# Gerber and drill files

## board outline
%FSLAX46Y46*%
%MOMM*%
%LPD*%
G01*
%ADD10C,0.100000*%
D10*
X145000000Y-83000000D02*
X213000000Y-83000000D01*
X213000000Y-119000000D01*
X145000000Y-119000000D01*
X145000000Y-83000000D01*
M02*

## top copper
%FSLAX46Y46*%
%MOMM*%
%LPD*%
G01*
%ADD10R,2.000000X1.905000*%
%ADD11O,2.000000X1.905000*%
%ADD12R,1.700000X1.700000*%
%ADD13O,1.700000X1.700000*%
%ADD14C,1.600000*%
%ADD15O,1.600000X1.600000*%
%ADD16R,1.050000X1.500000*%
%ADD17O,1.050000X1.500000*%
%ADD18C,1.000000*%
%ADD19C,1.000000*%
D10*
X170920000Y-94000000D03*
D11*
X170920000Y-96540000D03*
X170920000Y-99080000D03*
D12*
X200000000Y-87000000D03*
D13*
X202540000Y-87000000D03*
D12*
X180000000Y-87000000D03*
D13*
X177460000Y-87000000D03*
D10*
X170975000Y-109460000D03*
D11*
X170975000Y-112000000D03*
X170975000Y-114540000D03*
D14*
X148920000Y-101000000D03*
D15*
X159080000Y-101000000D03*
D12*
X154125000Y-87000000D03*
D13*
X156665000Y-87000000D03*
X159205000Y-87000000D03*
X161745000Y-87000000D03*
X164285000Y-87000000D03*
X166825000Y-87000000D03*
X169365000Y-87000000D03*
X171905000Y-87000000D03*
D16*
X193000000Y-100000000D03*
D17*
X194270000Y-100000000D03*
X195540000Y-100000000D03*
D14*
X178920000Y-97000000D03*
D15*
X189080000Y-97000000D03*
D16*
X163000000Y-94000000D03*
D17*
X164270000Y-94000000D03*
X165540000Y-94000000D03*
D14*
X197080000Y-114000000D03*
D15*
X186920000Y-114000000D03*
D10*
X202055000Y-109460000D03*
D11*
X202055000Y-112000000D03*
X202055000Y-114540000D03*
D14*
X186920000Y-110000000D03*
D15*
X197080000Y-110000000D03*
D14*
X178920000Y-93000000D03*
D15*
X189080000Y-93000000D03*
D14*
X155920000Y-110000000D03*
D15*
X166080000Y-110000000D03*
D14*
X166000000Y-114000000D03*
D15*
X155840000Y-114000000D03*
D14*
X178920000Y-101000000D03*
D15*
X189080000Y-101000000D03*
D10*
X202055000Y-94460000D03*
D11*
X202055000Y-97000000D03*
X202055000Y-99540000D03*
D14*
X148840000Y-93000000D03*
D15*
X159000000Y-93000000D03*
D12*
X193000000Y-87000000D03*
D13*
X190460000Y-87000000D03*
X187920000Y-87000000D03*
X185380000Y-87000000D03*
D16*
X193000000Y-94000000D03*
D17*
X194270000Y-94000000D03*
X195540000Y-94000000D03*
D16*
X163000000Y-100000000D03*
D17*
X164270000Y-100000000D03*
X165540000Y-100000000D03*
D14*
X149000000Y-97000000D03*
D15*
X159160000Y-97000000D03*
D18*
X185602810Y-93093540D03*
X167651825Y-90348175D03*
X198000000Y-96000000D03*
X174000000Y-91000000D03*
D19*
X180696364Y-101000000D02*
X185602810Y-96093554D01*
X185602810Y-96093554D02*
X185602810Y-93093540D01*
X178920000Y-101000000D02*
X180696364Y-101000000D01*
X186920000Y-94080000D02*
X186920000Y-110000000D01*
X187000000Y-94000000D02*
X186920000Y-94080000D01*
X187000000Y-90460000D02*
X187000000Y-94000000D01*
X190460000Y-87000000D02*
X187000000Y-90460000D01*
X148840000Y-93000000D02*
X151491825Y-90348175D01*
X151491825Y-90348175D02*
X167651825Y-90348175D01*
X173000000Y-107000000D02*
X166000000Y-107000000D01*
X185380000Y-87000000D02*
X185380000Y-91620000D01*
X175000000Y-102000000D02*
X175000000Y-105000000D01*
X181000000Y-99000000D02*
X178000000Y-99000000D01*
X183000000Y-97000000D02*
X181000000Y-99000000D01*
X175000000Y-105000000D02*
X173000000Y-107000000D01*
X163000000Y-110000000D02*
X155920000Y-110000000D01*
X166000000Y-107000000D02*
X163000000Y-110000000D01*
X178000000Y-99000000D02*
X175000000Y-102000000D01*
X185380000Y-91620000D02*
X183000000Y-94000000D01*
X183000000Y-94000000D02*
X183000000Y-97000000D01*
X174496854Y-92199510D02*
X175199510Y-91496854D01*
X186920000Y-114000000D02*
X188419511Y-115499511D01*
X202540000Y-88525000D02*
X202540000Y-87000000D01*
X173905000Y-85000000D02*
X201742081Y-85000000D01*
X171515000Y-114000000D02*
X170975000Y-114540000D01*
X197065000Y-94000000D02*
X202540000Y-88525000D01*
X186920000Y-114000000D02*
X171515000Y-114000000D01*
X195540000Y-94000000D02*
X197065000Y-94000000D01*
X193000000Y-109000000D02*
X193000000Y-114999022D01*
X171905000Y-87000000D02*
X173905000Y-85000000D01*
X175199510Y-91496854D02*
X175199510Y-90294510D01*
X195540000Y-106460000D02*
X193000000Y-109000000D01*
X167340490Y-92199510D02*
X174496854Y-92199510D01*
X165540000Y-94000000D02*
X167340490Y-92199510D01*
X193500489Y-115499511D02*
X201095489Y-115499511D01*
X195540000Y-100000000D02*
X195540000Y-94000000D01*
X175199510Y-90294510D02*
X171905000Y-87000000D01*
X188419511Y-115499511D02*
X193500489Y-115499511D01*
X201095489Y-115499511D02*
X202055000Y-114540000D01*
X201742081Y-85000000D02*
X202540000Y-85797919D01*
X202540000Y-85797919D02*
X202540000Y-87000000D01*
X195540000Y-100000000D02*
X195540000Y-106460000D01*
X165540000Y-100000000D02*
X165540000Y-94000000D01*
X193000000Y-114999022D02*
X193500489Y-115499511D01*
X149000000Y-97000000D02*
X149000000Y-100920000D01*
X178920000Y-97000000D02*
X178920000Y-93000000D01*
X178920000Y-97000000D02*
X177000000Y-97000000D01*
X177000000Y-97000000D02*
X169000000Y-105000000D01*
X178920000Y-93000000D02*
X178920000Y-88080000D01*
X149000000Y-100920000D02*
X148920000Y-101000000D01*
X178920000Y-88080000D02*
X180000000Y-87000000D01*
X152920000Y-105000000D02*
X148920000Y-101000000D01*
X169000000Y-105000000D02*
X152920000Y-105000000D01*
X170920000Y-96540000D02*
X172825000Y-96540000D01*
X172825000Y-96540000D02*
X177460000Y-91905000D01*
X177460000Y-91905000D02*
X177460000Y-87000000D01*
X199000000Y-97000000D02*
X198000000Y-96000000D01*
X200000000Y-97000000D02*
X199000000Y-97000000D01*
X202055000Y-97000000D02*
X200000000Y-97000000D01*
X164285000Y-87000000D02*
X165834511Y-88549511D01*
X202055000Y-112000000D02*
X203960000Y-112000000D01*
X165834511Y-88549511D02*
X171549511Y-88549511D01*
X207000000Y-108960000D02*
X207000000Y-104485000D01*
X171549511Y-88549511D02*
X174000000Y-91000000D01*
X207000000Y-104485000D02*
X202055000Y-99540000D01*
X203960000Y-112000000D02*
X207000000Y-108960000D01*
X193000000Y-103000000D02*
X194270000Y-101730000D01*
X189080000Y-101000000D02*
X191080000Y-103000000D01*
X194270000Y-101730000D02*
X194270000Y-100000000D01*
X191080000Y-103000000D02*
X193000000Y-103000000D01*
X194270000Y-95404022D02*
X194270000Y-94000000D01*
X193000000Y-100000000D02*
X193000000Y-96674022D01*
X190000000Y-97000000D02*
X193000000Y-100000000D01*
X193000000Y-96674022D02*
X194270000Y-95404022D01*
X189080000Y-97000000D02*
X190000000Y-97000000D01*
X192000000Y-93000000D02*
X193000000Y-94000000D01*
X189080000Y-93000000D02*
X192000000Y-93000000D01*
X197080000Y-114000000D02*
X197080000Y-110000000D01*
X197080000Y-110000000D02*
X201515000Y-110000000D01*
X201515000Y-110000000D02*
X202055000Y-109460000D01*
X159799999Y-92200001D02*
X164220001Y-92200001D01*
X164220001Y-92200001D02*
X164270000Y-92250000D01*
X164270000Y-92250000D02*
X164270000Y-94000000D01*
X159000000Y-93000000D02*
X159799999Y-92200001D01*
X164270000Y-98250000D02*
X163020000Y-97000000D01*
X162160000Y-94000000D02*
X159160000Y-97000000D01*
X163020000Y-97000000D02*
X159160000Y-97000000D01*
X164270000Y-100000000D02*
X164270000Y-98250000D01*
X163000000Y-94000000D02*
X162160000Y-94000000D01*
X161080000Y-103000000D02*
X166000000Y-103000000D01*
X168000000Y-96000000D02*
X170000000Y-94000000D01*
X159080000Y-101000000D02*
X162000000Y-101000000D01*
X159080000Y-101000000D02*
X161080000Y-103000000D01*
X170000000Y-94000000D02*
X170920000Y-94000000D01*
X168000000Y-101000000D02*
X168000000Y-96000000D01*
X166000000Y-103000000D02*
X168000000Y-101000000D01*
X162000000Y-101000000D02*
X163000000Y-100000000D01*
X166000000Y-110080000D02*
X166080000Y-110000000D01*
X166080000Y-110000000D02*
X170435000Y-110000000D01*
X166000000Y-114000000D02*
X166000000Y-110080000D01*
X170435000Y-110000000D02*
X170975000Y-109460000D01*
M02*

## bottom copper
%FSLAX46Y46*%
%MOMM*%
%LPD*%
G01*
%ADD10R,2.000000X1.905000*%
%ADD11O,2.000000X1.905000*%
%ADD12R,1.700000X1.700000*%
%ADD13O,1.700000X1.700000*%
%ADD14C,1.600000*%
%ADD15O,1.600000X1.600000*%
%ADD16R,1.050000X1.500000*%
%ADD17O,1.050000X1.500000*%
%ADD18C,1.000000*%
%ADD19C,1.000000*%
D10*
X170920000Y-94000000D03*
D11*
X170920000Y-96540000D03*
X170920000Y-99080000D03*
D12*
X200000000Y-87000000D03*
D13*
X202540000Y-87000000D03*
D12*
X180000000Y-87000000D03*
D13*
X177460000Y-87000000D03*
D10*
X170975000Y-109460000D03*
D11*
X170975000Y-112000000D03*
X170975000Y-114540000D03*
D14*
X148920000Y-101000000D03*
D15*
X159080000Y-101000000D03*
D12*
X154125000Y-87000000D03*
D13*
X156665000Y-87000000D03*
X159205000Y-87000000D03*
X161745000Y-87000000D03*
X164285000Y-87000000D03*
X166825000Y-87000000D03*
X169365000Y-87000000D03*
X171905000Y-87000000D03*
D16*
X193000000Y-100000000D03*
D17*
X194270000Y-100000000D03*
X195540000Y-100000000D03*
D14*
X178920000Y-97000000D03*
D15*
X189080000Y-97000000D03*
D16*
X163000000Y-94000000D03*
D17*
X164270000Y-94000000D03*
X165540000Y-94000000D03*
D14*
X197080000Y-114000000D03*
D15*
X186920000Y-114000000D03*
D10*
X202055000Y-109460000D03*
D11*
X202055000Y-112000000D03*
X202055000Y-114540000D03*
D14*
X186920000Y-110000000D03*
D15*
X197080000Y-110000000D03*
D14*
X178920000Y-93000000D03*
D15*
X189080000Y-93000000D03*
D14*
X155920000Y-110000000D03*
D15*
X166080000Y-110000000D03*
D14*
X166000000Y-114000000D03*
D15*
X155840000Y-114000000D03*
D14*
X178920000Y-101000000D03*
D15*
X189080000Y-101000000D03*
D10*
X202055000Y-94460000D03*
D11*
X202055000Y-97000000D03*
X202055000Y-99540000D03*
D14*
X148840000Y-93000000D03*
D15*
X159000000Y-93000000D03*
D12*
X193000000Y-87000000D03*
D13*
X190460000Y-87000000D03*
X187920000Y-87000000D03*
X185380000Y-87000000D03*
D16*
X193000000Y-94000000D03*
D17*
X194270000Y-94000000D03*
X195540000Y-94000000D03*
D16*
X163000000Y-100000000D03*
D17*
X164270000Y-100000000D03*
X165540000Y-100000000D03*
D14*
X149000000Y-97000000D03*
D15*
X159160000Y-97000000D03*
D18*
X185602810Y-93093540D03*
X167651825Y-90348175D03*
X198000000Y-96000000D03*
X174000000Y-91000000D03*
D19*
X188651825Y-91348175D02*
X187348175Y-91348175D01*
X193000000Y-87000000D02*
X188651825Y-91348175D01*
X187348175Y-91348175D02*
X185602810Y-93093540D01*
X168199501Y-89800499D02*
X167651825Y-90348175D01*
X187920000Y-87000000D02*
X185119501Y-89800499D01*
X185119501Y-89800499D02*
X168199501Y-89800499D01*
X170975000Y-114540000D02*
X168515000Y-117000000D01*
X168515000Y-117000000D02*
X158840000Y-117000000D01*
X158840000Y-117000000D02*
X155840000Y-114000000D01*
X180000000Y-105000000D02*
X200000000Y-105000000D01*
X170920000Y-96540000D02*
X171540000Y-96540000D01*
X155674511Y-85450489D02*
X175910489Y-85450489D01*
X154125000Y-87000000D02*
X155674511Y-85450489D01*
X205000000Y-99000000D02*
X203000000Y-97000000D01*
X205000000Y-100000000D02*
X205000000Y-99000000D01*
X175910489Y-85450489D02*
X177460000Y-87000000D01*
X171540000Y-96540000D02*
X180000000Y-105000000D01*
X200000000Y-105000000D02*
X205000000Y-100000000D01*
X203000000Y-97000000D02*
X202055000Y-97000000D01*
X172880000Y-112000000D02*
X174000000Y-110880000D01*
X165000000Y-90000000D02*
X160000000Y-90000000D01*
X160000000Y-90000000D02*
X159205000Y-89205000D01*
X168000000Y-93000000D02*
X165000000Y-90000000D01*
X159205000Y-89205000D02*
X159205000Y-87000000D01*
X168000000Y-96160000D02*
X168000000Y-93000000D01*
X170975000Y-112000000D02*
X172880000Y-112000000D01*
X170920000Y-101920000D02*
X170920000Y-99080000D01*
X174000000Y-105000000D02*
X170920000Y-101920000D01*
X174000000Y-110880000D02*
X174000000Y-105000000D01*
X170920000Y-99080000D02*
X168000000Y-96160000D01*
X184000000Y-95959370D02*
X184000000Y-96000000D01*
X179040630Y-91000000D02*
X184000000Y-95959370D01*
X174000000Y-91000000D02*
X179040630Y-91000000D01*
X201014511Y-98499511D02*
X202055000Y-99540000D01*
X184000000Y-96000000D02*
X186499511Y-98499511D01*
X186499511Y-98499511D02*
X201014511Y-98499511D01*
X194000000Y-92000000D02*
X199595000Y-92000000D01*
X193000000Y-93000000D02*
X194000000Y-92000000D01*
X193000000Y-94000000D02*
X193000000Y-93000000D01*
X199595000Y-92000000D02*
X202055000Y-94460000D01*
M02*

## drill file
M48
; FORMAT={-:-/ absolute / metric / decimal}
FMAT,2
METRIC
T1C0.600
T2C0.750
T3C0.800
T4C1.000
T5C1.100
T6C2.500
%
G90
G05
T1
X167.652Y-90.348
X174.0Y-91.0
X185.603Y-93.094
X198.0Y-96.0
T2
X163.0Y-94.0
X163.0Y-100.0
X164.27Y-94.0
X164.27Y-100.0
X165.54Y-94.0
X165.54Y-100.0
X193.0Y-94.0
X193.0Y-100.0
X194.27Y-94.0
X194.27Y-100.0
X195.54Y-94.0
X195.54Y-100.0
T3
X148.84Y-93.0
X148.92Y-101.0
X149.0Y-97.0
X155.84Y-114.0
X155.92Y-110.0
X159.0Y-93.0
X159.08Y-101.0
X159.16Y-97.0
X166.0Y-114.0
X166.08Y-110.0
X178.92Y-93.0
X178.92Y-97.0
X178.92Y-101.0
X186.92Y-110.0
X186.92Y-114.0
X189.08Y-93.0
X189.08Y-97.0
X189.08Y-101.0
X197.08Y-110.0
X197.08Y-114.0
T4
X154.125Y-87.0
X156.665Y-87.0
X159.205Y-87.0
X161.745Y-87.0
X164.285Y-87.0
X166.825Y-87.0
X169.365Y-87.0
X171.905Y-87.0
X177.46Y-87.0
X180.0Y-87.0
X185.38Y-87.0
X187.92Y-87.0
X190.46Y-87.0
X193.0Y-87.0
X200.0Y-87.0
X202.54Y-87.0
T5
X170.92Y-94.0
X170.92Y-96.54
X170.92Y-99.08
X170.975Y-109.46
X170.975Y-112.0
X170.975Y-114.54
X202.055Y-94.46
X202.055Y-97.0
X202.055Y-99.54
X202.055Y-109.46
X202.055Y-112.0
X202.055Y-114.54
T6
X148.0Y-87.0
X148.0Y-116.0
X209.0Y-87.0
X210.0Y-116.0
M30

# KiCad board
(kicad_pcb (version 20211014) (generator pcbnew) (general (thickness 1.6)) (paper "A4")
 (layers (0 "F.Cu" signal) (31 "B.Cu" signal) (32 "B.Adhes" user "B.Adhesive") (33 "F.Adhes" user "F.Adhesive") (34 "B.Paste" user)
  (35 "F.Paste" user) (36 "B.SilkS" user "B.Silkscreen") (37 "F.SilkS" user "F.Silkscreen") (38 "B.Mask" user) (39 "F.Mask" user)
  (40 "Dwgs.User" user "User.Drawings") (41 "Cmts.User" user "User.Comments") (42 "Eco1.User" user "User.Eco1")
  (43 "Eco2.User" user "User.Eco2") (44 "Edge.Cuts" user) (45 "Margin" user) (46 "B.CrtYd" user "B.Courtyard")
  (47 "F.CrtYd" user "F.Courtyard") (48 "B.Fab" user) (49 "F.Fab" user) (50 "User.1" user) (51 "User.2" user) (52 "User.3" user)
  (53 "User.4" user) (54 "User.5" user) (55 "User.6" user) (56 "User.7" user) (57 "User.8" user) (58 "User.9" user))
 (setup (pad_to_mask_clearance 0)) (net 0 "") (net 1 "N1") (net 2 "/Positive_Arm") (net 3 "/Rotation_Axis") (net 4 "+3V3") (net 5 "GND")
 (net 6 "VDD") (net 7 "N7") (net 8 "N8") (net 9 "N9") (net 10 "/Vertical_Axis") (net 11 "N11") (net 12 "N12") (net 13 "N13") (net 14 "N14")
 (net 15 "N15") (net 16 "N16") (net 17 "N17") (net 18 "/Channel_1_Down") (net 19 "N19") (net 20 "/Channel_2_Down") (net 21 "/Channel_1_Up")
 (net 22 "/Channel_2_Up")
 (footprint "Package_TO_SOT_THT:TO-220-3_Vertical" (layer "F.Cu") (at 170.92 94 -90)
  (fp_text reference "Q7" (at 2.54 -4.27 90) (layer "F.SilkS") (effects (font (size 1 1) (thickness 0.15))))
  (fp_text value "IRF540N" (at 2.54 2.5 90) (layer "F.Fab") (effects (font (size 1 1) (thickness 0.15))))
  (pad "1" thru_hole rect locked (at 0 0 270) (size 1.905 2) (drill 1.1) (layers *.Cu *.Mask) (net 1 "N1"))
  (pad "2" thru_hole oval locked (at 2.54 0 270) (size 1.905 2) (drill 1.1) (layers *.Cu *.Mask) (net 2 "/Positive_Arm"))
  (pad "3" thru_hole oval locked (at 5.08 0 270) (size 1.905 2) (drill 1.1) (layers *.Cu *.Mask) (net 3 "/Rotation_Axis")))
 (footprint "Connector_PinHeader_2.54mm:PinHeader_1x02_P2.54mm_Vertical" (layer "F.Cu") (at 200 87 90)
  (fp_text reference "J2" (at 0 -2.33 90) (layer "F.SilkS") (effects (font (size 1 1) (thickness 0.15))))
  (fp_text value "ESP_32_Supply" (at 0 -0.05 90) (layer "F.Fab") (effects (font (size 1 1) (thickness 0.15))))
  (pad "1" thru_hole rect locked (at 0 0 90) (size 1.7 1.7) (drill 1) (layers *.Cu *.Mask) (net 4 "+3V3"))
  (pad "2" thru_hole oval locked (at 0 2.54 90) (size 1.7 1.7) (drill 1) (layers *.Cu *.Mask) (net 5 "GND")))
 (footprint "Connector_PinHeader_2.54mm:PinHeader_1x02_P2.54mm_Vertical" (layer "F.Cu") (at 180 87 -90)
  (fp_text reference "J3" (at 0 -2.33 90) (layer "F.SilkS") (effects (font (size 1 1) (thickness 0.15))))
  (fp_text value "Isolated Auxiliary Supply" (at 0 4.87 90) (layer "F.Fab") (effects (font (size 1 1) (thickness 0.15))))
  (pad "1" thru_hole rect locked (at 0 0 270) (size 1.7 1.7) (drill 1) (layers *.Cu *.Mask) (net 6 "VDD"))
  (pad "2" thru_hole oval locked (at 0 2.54 270) (size 1.7 1.7) (drill 1) (layers *.Cu *.Mask) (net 2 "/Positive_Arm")))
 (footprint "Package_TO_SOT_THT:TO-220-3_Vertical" (layer "F.Cu") (at 170.975 109.46 -90)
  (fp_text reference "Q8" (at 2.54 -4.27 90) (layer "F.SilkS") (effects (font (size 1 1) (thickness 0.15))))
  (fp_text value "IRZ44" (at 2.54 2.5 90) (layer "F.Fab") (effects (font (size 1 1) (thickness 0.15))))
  (pad "1" thru_hole rect locked (at 0 0 270) (size 1.905 2) (drill 1.1) (layers *.Cu *.Mask) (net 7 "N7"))
  (pad "2" thru_hole oval locked (at 2.54 0 270) (size 1.905 2) (drill 1.1) (layers *.Cu *.Mask) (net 3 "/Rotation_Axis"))
  (pad "3" thru_hole oval locked (at 5.08 0 270) (size 1.905 2) (drill 1.1) (layers *.Cu *.Mask) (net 5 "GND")))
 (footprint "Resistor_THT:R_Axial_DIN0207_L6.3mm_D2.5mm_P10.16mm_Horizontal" (layer "F.Cu") (at 148.92 101)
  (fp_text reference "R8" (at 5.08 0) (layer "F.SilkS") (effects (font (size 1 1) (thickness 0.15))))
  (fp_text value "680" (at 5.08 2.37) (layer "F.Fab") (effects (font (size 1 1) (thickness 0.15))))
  (pad "1" thru_hole circle locked (at 0 0) (size 1.6 1.6) (drill 0.8) (layers *.Cu *.Mask) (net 6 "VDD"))
  (pad "2" thru_hole oval locked (at 10.16 0) (size 1.6 1.6) (drill 0.8) (layers *.Cu *.Mask) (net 1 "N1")))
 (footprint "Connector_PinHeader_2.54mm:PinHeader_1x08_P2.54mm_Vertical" (layer "F.Cu") (at 154.125 87 90)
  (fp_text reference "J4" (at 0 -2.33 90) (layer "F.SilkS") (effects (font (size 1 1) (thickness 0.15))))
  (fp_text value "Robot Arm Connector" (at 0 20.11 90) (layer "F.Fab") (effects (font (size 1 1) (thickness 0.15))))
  (pad "1" thru_hole rect locked (at 0 0 90) (size 1.7 1.7) (drill 1) (layers *.Cu *.Mask) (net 2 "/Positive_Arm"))
  (pad "2" thru_hole oval locked (at 0 2.54 90) (size 1.7 1.7) (drill 1) (layers *.Cu *.Mask) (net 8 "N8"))
  (pad "3" thru_hole oval locked (at 0 5.08 90) (size 1.7 1.7) (drill 1) (layers *.Cu *.Mask) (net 3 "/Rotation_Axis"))
  (pad "4" thru_hole oval locked (at 0 7.62 90) (size 1.7 1.7) (drill 1) (layers *.Cu *.Mask) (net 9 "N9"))
  (pad "5" thru_hole oval locked (at 0 10.16 90) (size 1.7 1.7) (drill 1) (layers *.Cu *.Mask) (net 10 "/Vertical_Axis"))
  (pad "6" thru_hole oval locked (at 0 12.7 90) (size 1.7 1.7) (drill 1) (layers *.Cu *.Mask) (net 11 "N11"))
  (pad "7" thru_hole oval locked (at 0 15.24 90) (size 1.7 1.7) (drill 1) (layers *.Cu *.Mask) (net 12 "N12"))
  (pad "8" thru_hole oval locked (at 0 17.78 90) (size 1.7 1.7) (drill 1) (layers *.Cu *.Mask) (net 5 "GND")))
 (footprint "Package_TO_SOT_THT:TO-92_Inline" (layer "F.Cu") (at 193 100)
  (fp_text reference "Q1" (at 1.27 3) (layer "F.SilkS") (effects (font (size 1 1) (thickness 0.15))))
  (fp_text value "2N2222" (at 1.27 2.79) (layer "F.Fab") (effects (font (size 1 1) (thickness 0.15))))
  (pad "1" thru_hole rect locked (at 0 0) (size 1.05 1.5) (drill 0.75) (layers *.Cu *.Mask) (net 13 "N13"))
  (pad "2" thru_hole oval locked (at 1.27 0) (size 1.05 1.5) (drill 0.75) (layers *.Cu *.Mask) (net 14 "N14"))
  (pad "3" thru_hole oval locked (at 2.54 0) (size 1.05 1.5) (drill 0.75) (layers *.Cu *.Mask) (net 5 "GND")))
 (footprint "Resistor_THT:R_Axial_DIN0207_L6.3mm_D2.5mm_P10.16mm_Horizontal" (layer "F.Cu") (at 178.92 97)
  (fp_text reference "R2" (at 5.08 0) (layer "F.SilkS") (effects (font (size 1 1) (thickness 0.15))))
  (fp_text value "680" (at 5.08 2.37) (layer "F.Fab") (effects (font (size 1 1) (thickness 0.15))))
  (pad "1" thru_hole circle locked (at 0 0) (size 1.6 1.6) (drill 0.8) (layers *.Cu *.Mask) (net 6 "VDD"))
  (pad "2" thru_hole oval locked (at 10.16 0) (size 1.6 1.6) (drill 0.8) (layers *.Cu *.Mask) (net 13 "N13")))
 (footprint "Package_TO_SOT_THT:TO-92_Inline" (layer "F.Cu") (at 163 94)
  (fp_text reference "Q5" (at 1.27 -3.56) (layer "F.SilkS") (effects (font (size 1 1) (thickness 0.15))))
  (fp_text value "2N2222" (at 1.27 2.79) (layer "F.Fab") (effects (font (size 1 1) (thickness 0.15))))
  (pad "1" thru_hole rect locked (at 0 0) (size 1.05 1.5) (drill 0.75) (layers *.Cu *.Mask) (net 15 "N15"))
  (pad "2" thru_hole oval locked (at 1.27 0) (size 1.05 1.5) (drill 0.75) (layers *.Cu *.Mask) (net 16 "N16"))
  (pad "3" thru_hole oval locked (at 2.54 0) (size 1.05 1.5) (drill 0.75) (layers *.Cu *.Mask) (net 5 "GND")))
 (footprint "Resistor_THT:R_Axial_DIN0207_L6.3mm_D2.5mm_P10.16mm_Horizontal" (layer "F.Cu") (at 197.08 114 180)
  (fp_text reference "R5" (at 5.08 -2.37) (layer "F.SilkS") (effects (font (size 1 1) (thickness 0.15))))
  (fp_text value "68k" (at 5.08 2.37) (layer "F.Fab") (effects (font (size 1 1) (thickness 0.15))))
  (pad "1" thru_hole circle locked (at 0 0 180) (size 1.6 1.6) (drill 0.8) (layers *.Cu *.Mask) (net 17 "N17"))
  (pad "2" thru_hole oval locked (at 10.16 0 180) (size 1.6 1.6) (drill 0.8) (layers *.Cu *.Mask) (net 5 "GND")))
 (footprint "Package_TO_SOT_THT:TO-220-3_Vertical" (layer "F.Cu") (at 202.055 109.46 -90)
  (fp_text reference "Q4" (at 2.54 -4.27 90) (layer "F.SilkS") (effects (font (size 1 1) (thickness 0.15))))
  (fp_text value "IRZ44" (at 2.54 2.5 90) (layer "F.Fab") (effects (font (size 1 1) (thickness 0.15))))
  (pad "1" thru_hole rect locked (at 0 0 270) (size 1.905 2) (drill 1.1) (layers *.Cu *.Mask) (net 17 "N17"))
  (pad "2" thru_hole oval locked (at 2.54 0 270) (size 1.905 2) (drill 1.1) (layers *.Cu *.Mask) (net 10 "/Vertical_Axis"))
  (pad "3" thru_hole oval locked (at 5.08 0 270) (size 1.905 2) (drill 1.1) (layers *.Cu *.Mask) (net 5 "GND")))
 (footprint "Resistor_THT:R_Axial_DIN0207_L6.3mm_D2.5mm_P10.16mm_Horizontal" (layer "F.Cu") (at 186.92 110)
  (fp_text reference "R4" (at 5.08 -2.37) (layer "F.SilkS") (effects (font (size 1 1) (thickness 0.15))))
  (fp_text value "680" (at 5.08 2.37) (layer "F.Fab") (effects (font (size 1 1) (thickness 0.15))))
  (pad "1" thru_hole circle locked (at 0 0) (size 1.6 1.6) (drill 0.8) (layers *.Cu *.Mask) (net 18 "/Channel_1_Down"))
  (pad "2" thru_hole oval locked (at 10.16 0) (size 1.6 1.6) (drill 0.8) (layers *.Cu *.Mask) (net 17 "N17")))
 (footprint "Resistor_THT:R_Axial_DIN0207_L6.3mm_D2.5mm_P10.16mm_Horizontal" (layer "F.Cu") (at 178.92 93)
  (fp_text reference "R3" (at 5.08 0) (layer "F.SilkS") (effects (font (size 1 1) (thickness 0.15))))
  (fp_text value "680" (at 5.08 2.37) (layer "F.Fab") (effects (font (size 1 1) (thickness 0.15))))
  (pad "1" thru_hole circle locked (at 0 0) (size 1.6 1.6) (drill 0.8) (layers *.Cu *.Mask) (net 6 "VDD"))
  (pad "2" thru_hole oval locked (at 10.16 0) (size 1.6 1.6) (drill 0.8) (layers *.Cu *.Mask) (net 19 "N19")))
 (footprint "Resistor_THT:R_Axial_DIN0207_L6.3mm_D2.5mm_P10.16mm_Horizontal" (layer "F.Cu") (at 155.92 110)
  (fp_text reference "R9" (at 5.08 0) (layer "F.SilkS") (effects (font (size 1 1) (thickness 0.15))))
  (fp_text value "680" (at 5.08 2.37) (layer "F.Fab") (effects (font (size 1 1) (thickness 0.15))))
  (pad "1" thru_hole circle locked (at 0 0) (size 1.6 1.6) (drill 0.8) (layers *.Cu *.Mask) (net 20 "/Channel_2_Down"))
  (pad "2" thru_hole oval locked (at 10.16 0) (size 1.6 1.6) (drill 0.8) (layers *.Cu *.Mask) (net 7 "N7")))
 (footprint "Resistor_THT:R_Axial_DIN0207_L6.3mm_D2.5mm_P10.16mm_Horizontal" (layer "F.Cu") (at 166 114 180)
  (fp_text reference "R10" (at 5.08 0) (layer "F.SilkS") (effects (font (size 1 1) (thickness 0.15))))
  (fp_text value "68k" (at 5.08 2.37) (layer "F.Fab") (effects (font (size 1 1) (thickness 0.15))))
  (pad "1" thru_hole circle locked (at 0 0 180) (size 1.6 1.6) (drill 0.8) (layers *.Cu *.Mask) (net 7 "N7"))
  (pad "2" thru_hole oval locked (at 10.16 0 180) (size 1.6 1.6) (drill 0.8) (layers *.Cu *.Mask) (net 5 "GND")))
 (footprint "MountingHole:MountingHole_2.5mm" (layer "F.Cu") (at 148 87)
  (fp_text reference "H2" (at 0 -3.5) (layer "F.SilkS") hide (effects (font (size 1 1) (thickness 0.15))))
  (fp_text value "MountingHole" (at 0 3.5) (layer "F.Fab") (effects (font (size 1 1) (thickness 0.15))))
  (pad "" np_thru_hole circle locked (at 0 0) (size 2.5 2.5) (drill 2.5) (layers *.Cu *.Mask)))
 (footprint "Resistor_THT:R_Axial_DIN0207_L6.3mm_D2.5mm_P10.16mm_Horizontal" (layer "F.Cu") (at 178.92 101)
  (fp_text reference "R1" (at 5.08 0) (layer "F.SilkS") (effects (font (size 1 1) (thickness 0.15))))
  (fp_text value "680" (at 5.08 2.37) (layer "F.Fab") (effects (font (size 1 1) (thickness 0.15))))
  (pad "1" thru_hole circle locked (at 0 0) (size 1.6 1.6) (drill 0.8) (layers *.Cu *.Mask) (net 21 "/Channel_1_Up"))
  (pad "2" thru_hole oval locked (at 10.16 0) (size 1.6 1.6) (drill 0.8) (layers *.Cu *.Mask) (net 14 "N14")))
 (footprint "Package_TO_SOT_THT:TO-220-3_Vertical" (layer "F.Cu") (at 202.055 94.46 -90)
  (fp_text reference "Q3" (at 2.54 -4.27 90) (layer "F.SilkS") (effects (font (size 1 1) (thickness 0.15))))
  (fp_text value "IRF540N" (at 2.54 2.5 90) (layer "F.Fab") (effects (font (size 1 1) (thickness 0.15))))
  (pad "1" thru_hole rect locked (at 0 0 270) (size 1.905 2) (drill 1.1) (layers *.Cu *.Mask) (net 19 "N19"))
  (pad "2" thru_hole oval locked (at 2.54 0 270) (size 1.905 2) (drill 1.1) (layers *.Cu *.Mask) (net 2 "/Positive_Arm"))
  (pad "3" thru_hole oval locked (at 5.08 0 270) (size 1.905 2) (drill 1.1) (layers *.Cu *.Mask) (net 10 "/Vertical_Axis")))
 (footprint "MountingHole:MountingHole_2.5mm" (layer "F.Cu") (at 210 116)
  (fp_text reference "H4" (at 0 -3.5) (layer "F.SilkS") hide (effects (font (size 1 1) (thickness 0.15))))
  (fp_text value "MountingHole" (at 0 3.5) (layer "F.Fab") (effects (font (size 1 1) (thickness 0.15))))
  (pad "" np_thru_hole circle locked (at 0 0) (size 2.5 2.5) (drill 2.5) (layers *.Cu *.Mask)))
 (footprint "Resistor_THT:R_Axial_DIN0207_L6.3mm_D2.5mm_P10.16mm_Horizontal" (layer "F.Cu") (at 148.84 93)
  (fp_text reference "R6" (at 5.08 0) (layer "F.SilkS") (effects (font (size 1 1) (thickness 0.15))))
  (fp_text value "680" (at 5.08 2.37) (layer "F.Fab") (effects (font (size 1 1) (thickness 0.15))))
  (pad "1" thru_hole circle locked (at 0 0) (size 1.6 1.6) (drill 0.8) (layers *.Cu *.Mask) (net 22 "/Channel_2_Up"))
  (pad "2" thru_hole oval locked (at 10.16 0) (size 1.6 1.6) (drill 0.8) (layers *.Cu *.Mask) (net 16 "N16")))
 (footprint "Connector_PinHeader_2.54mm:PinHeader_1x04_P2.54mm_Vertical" (layer "F.Cu") (at 193 87 -90)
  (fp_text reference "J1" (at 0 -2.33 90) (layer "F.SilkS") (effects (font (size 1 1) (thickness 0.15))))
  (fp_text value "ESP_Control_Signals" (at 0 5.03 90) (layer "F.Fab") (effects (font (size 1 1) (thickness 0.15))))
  (pad "1" thru_hole rect locked (at 0 0 270) (size 1.7 1.7) (drill 1) (layers *.Cu *.Mask) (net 21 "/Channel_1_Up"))
  (pad "2" thru_hole oval locked (at 0 2.54 270) (size 1.7 1.7) (drill 1) (layers *.Cu *.Mask) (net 18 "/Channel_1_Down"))
  (pad "3" thru_hole oval locked (at 0 5.08 270) (size 1.7 1.7) (drill 1) (layers *.Cu *.Mask) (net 22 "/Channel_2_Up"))
  (pad "4" thru_hole oval locked (at 0 7.62 270) (size 1.7 1.7) (drill 1) (layers *.Cu *.Mask) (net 20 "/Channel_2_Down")))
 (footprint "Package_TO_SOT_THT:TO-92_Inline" (layer "F.Cu") (at 193 94)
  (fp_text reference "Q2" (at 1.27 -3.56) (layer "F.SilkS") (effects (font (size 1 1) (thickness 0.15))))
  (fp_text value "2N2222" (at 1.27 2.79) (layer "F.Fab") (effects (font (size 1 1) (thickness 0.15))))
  (pad "1" thru_hole rect locked (at 0 0) (size 1.05 1.5) (drill 0.75) (layers *.Cu *.Mask) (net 19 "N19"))
  (pad "2" thru_hole oval locked (at 1.27 0) (size 1.05 1.5) (drill 0.75) (layers *.Cu *.Mask) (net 13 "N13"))
  (pad "3" thru_hole oval locked (at 2.54 0) (size 1.05 1.5) (drill 0.75) (layers *.Cu *.Mask) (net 5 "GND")))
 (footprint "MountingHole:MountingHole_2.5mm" (layer "F.Cu") (at 209 87)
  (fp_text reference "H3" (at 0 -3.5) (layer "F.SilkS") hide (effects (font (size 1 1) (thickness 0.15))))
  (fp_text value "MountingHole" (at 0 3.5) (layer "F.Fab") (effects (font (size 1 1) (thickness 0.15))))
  (pad "" np_thru_hole circle locked (at 0 0) (size 2.5 2.5) (drill 2.5) (layers *.Cu *.Mask)))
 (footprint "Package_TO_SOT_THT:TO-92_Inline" (layer "F.Cu") (at 163 100)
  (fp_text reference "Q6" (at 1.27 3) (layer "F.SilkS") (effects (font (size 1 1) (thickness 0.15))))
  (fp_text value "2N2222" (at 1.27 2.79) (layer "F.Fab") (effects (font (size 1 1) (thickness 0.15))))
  (pad "1" thru_hole rect locked (at 0 0) (size 1.05 1.5) (drill 0.75) (layers *.Cu *.Mask) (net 1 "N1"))
  (pad "2" thru_hole oval locked (at 1.27 0) (size 1.05 1.5) (drill 0.75) (layers *.Cu *.Mask) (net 15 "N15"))
  (pad "3" thru_hole oval locked (at 2.54 0) (size 1.05 1.5) (drill 0.75) (layers *.Cu *.Mask) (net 5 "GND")))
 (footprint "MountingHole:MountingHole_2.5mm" (layer "F.Cu") (at 148 116)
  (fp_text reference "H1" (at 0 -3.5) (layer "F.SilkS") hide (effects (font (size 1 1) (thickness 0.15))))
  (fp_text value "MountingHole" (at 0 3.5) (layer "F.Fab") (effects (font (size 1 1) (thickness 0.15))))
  (pad "" np_thru_hole circle locked (at 0 0) (size 2.5 2.5) (drill 2.5) (layers *.Cu *.Mask)))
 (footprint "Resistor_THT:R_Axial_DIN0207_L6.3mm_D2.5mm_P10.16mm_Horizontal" (layer "F.Cu") (at 149 97)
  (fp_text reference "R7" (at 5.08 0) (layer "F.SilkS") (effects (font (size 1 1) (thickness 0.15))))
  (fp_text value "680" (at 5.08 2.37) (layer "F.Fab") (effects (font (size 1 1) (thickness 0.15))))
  (pad "1" thru_hole circle locked (at 0 0) (size 1.6 1.6) (drill 0.8) (layers *.Cu *.Mask) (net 6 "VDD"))
  (pad "2" thru_hole oval locked (at 10.16 0) (size 1.6 1.6) (drill 0.8) (layers *.Cu *.Mask) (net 15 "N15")))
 (gr_rect (start 145 83) (end 213 119) (layer "Edge.Cuts") (width 0.1) (fill none))
 (segment (start 180.696364 101) (end 185.60281 96.093554) (width 1) (layer "F.Cu") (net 21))
 (segment (start 185.60281 96.093554) (end 185.60281 93.09354) (width 1) (layer "F.Cu") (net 21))
 (segment (start 178.92 101) (end 180.696364 101) (width 1) (layer "F.Cu") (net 21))
 (via (at 185.60281 93.09354) (size 1) (drill 0.6) (layers "F.Cu" "B.Cu") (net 21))
 (segment (start 188.651825 91.348175) (end 187.348175 91.348175) (width 1) (layer "B.Cu") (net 21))
 (segment (start 193 87) (end 188.651825 91.348175) (width 1) (layer "B.Cu") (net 21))
 (segment (start 187.348175 91.348175) (end 185.60281 93.09354) (width 1) (layer "B.Cu") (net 21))
 (segment (start 186.92 94.08) (end 186.92 110) (width 1) (layer "F.Cu") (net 18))
 (segment (start 187 94) (end 186.92 94.08) (width 1) (layer "F.Cu") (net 18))
 (segment (start 187 90.46) (end 187 94) (width 1) (layer "F.Cu") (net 18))
 (segment (start 190.46 87) (end 187 90.46) (width 1) (layer "F.Cu") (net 18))
 (segment (start 148.84 93) (end 151.491825 90.348175) (width 1) (layer "F.Cu") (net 22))
 (segment (start 151.491825 90.348175) (end 167.651825 90.348175) (width 1) (layer "F.Cu") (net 22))
 (via (at 167.651825 90.348175) (size 1) (drill 0.6) (layers "F.Cu" "B.Cu") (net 22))
 (segment (start 168.199501 89.800499) (end 167.651825 90.348175) (width 1) (layer "B.Cu") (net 22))
 (segment (start 187.92 87) (end 185.119501 89.800499) (width 1) (layer "B.Cu") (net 22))
 (segment (start 185.119501 89.800499) (end 168.199501 89.800499) (width 1) (layer "B.Cu") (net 22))
 (segment (start 173 107) (end 166 107) (width 1) (layer "F.Cu") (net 20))
 (segment (start 185.38 87) (end 185.38 91.62) (width 1) (layer "F.Cu") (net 20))
 (segment (start 175 102) (end 175 105) (width 1) (layer "F.Cu") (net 20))
 (segment (start 181 99) (end 178 99) (width 1) (layer "F.Cu") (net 20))
 (segment (start 183 97) (end 181 99) (width 1) (layer "F.Cu") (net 20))
 (segment (start 175 105) (end 173 107) (width 1) (layer "F.Cu") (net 20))
 (segment (start 163 110) (end 155.92 110) (width 1) (layer "F.Cu") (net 20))
 (segment (start 166 107) (end 163 110) (width 1) (layer "F.Cu") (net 20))
 (segment (start 178 99) (end 175 102) (width 1) (layer "F.Cu") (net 20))
 (segment (start 185.38 91.62) (end 183 94) (width 1) (layer "F.Cu") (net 20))
 (segment (start 183 94) (end 183 97) (width 1) (layer "F.Cu") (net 20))
 (segment (start 174.496854 92.19951) (end 175.19951 91.496854) (width 1) (layer "F.Cu") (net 5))
 (segment (start 186.92 114) (end 188.419511 115.499511) (width 1) (layer "F.Cu") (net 5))
 (segment (start 202.54 88.525) (end 202.54 87) (width 1) (layer "F.Cu") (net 5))
 (segment (start 173.905 85) (end 201.742081 85) (width 1) (layer "F.Cu") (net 5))
 (segment (start 171.515 114) (end 170.975 114.54) (width 1) (layer "F.Cu") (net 5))
 (segment (start 197.065 94) (end 202.54 88.525) (width 1) (layer "F.Cu") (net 5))
 (segment (start 186.92 114) (end 171.515 114) (width 1) (layer "F.Cu") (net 5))
 (segment (start 195.54 94) (end 197.065 94) (width 1) (layer "F.Cu") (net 5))
 (segment (start 193 109) (end 193 114.999022) (width 1) (layer "F.Cu") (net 5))
 (segment (start 171.905 87) (end 173.905 85) (width 1) (layer "F.Cu") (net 5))
 (segment (start 175.19951 91.496854) (end 175.19951 90.29451) (width 1) (layer "F.Cu") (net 5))
 (segment (start 195.54 106.46) (end 193 109) (width 1) (layer "F.Cu") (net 5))
 (segment (start 167.34049 92.19951) (end 174.496854 92.19951) (width 1) (layer "F.Cu") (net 5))
 (segment (start 165.54 94) (end 167.34049 92.19951) (width 1) (layer "F.Cu") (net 5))
 (segment (start 193.500489 115.499511) (end 201.095489 115.499511) (width 1) (layer "F.Cu") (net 5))
 (segment (start 195.54 100) (end 195.54 94) (width 1) (layer "F.Cu") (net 5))
 (segment (start 175.19951 90.29451) (end 171.905 87) (width 1) (layer "F.Cu") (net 5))
 (segment (start 188.419511 115.499511) (end 193.500489 115.499511) (width 1) (layer "F.Cu") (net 5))
 (segment (start 201.095489 115.499511) (end 202.055 114.54) (width 1) (layer "F.Cu") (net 5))
 (segment (start 201.742081 85) (end 202.54 85.797919) (width 1) (layer "F.Cu") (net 5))
 (segment (start 202.54 85.797919) (end 202.54 87) (width 1) (layer "F.Cu") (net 5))
 (segment (start 195.54 100) (end 195.54 106.46) (width 1) (layer "F.Cu") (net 5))
 (segment (start 165.54 100) (end 165.54 94) (width 1) (layer "F.Cu") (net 5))
 (segment (start 193 114.999022) (end 193.500489 115.499511) (width 1) (layer "F.Cu") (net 5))
 (segment (start 170.975 114.54) (end 168.515 117) (width 1) (layer "B.Cu") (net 5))
 (segment (start 168.515 117) (end 158.84 117) (width 1) (layer "B.Cu") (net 5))
 (segment (start 158.84 117) (end 155.84 114) (width 1) (layer "B.Cu") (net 5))
 (segment (start 149 97) (end 149 100.92) (width 1) (layer "F.Cu") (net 6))
 (segment (start 178.92 97) (end 178.92 93) (width 1) (layer "F.Cu") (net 6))
 (segment (start 178.92 97) (end 177 97) (width 1) (layer "F.Cu") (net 6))
 (segment (start 177 97) (end 169 105) (width 1) (layer "F.Cu") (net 6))
 (segment (start 178.92 93) (end 178.92 88.08) (width 1) (layer "F.Cu") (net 6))
 (segment (start 149 100.92) (end 148.92 101) (width 1) (layer "F.Cu") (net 6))
 (segment (start 178.92 88.08) (end 180 87) (width 1) (layer "F.Cu") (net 6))
 (segment (start 152.92 105) (end 148.92 101) (width 1) (layer "F.Cu") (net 6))
 (segment (start 169 105) (end 152.92 105) (width 1) (layer "F.Cu") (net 6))
 (segment (start 170.92 96.54) (end 172.825 96.54) (width 1) (layer "F.Cu") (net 2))
 (segment (start 172.825 96.54) (end 177.46 91.905) (width 1) (layer "F.Cu") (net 2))
 (segment (start 177.46 91.905) (end 177.46 87) (width 1) (layer "F.Cu") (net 2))
 (segment (start 199 97) (end 198 96) (width 1) (layer "F.Cu") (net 2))
 (segment (start 200 97) (end 199 97) (width 1) (layer "F.Cu") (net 2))
 (segment (start 202.055 97) (end 200 97) (width 1) (layer "F.Cu") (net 2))
 (via (at 198 96) (size 1) (drill 0.6) (layers "F.Cu" "B.Cu") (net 2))
 (segment (start 180 105) (end 200 105) (width 1) (layer "B.Cu") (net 2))
 (segment (start 170.92 96.54) (end 171.54 96.54) (width 1) (layer "B.Cu") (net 2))
 (segment (start 155.674511 85.450489) (end 175.910489 85.450489) (width 1) (layer "B.Cu") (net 2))
 (segment (start 154.125 87) (end 155.674511 85.450489) (width 1) (layer "B.Cu") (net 2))
 (segment (start 205 99) (end 203 97) (width 1) (layer "B.Cu") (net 2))
 (segment (start 205 100) (end 205 99) (width 1) (layer "B.Cu") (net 2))
 (segment (start 175.910489 85.450489) (end 177.46 87) (width 1) (layer "B.Cu") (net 2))
 (segment (start 171.54 96.54) (end 180 105) (width 1) (layer "B.Cu") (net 2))
 (segment (start 200 105) (end 205 100) (width 1) (layer "B.Cu") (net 2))
 (segment (start 203 97) (end 202.055 97) (width 1) (layer "B.Cu") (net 2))
 (segment (start 172.88 112) (end 174 110.88) (width 1) (layer "B.Cu") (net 3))
 (segment (start 165 90) (end 160 90) (width 1) (layer "B.Cu") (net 3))
 (segment (start 160 90) (end 159.205 89.205) (width 1) (layer "B.Cu") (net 3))
 (segment (start 168 93) (end 165 90) (width 1) (layer "B.Cu") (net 3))
 (segment (start 159.205 89.205) (end 159.205 87) (width 1) (layer "B.Cu") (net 3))
 (segment (start 168 96.16) (end 168 93) (width 1) (layer "B.Cu") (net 3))
 (segment (start 170.975 112) (end 172.88 112) (width 1) (layer "B.Cu") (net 3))
 (segment (start 170.92 101.92) (end 170.92 99.08) (width 1) (layer "B.Cu") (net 3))
 (segment (start 174 105) (end 170.92 101.92) (width 1) (layer "B.Cu") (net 3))
 (segment (start 174 110.88) (end 174 105) (width 1) (layer "B.Cu") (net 3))
 (segment (start 170.92 99.08) (end 168 96.16) (width 1) (layer "B.Cu") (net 3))
 (segment (start 164.285 87) (end 165.834511 88.549511) (width 1) (layer "F.Cu") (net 10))
 (segment (start 202.055 112) (end 203.96 112) (width 1) (layer "F.Cu") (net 10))
 (segment (start 165.834511 88.549511) (end 171.549511 88.549511) (width 1) (layer "F.Cu") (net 10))
 (segment (start 207 108.96) (end 207 104.485) (width 1) (layer "F.Cu") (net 10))
 (segment (start 171.549511 88.549511) (end 174 91) (width 1) (layer "F.Cu") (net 10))
 (segment (start 207 104.485) (end 202.055 99.54) (width 1) (layer "F.Cu") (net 10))
 (segment (start 203.96 112) (end 207 108.96) (width 1) (layer "F.Cu") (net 10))
 (via (at 174 91) (size 1) (drill 0.6) (layers "F.Cu" "B.Cu") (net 10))
 (segment (start 184 95.95937) (end 184 96) (width 1) (layer "B.Cu") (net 10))
 (segment (start 179.04063 91) (end 184 95.95937) (width 1) (layer "B.Cu") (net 10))
 (segment (start 174 91) (end 179.04063 91) (width 1) (layer "B.Cu") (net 10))
 (segment (start 201.014511 98.499511) (end 202.055 99.54) (width 1) (layer "B.Cu") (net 10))
 (segment (start 184 96) (end 186.499511 98.499511) (width 1) (layer "B.Cu") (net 10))
 (segment (start 186.499511 98.499511) (end 201.014511 98.499511) (width 1) (layer "B.Cu") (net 10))
 (segment (start 193 103) (end 194.27 101.73) (width 1) (layer "F.Cu") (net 14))
 (segment (start 189.08 101) (end 191.08 103) (width 1) (layer "F.Cu") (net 14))
 (segment (start 194.27 101.73) (end 194.27 100) (width 1) (layer "F.Cu") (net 14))
 (segment (start 191.08 103) (end 193 103) (width 1) (layer "F.Cu") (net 14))
 (segment (start 194.27 95.404022) (end 194.27 94) (width 1) (layer "F.Cu") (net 13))
 (segment (start 193 100) (end 193 96.674022) (width 1) (layer "F.Cu") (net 13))
 (segment (start 190 97) (end 193 100) (width 1) (layer "F.Cu") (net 13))
 (segment (start 193 96.674022) (end 194.27 95.404022) (width 1) (layer "F.Cu") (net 13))
 (segment (start 189.08 97) (end 190 97) (width 1) (layer "F.Cu") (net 13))
 (segment (start 192 93) (end 193 94) (width 1) (layer "F.Cu") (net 19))
 (segment (start 189.08 93) (end 192 93) (width 1) (layer "F.Cu") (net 19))
 (segment (start 194 92) (end 199.595 92) (width 1) (layer "B.Cu") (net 19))
 (segment (start 193 93) (end 194 92) (width 1) (layer "B.Cu") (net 19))
 (segment (start 193 94) (end 193 93) (width 1) (layer "B.Cu") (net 19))
 (segment (start 199.595 92) (end 202.055 94.46) (width 1) (layer "B.Cu") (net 19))
 (segment (start 197.08 114) (end 197.08 110) (width 1) (layer "F.Cu") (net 17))
 (segment (start 197.08 110) (end 201.515 110) (width 1) (layer "F.Cu") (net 17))
 (segment (start 201.515 110) (end 202.055 109.46) (width 1) (layer "F.Cu") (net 17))
 (segment (start 159.799999 92.200001) (end 164.220001 92.200001) (width 1) (layer "F.Cu") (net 16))
 (segment (start 164.220001 92.200001) (end 164.27 92.25) (width 1) (layer "F.Cu") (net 16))
 (segment (start 164.27 92.25) (end 164.27 94) (width 1) (layer "F.Cu") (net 16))
 (segment (start 159 93) (end 159.799999 92.200001) (width 1) (layer "F.Cu") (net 16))
 (segment (start 164.27 98.25) (end 163.02 97) (width 1) (layer "F.Cu") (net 15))
 (segment (start 162.16 94) (end 159.16 97) (width 1) (layer "F.Cu") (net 15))
 (segment (start 163.02 97) (end 159.16 97) (width 1) (layer "F.Cu") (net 15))
 (segment (start 164.27 100) (end 164.27 98.25) (width 1) (layer "F.Cu") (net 15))
 (segment (start 163 94) (end 162.16 94) (width 1) (layer "F.Cu") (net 15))
 (segment (start 161.08 103) (end 166 103) (width 1) (layer "F.Cu") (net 1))
 (segment (start 168 96) (end 170 94) (width 1) (layer "F.Cu") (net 1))
 (segment (start 159.08 101) (end 162 101) (width 1) (layer "F.Cu") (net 1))
 (segment (start 159.08 101) (end 161.08 103) (width 1) (layer "F.Cu") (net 1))
 (segment (start 170 94) (end 170.92 94) (width 1) (layer "F.Cu") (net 1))
 (segment (start 168 101) (end 168 96) (width 1) (layer "F.Cu") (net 1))
 (segment (start 166 103) (end 168 101) (width 1) (layer "F.Cu") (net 1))
 (segment (start 162 101) (end 163 100) (width 1) (layer "F.Cu") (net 1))
 (segment (start 166 110.08) (end 166.08 110) (width 1) (layer "F.Cu") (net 7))
 (segment (start 166.08 110) (end 170.435 110) (width 1) (layer "F.Cu") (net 7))
 (segment (start 166 114) (end 166 110.08) (width 1) (layer "F.Cu") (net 7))
 (segment (start 170.435 110) (end 170.975 109.46) (width 1) (layer "F.Cu") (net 7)))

